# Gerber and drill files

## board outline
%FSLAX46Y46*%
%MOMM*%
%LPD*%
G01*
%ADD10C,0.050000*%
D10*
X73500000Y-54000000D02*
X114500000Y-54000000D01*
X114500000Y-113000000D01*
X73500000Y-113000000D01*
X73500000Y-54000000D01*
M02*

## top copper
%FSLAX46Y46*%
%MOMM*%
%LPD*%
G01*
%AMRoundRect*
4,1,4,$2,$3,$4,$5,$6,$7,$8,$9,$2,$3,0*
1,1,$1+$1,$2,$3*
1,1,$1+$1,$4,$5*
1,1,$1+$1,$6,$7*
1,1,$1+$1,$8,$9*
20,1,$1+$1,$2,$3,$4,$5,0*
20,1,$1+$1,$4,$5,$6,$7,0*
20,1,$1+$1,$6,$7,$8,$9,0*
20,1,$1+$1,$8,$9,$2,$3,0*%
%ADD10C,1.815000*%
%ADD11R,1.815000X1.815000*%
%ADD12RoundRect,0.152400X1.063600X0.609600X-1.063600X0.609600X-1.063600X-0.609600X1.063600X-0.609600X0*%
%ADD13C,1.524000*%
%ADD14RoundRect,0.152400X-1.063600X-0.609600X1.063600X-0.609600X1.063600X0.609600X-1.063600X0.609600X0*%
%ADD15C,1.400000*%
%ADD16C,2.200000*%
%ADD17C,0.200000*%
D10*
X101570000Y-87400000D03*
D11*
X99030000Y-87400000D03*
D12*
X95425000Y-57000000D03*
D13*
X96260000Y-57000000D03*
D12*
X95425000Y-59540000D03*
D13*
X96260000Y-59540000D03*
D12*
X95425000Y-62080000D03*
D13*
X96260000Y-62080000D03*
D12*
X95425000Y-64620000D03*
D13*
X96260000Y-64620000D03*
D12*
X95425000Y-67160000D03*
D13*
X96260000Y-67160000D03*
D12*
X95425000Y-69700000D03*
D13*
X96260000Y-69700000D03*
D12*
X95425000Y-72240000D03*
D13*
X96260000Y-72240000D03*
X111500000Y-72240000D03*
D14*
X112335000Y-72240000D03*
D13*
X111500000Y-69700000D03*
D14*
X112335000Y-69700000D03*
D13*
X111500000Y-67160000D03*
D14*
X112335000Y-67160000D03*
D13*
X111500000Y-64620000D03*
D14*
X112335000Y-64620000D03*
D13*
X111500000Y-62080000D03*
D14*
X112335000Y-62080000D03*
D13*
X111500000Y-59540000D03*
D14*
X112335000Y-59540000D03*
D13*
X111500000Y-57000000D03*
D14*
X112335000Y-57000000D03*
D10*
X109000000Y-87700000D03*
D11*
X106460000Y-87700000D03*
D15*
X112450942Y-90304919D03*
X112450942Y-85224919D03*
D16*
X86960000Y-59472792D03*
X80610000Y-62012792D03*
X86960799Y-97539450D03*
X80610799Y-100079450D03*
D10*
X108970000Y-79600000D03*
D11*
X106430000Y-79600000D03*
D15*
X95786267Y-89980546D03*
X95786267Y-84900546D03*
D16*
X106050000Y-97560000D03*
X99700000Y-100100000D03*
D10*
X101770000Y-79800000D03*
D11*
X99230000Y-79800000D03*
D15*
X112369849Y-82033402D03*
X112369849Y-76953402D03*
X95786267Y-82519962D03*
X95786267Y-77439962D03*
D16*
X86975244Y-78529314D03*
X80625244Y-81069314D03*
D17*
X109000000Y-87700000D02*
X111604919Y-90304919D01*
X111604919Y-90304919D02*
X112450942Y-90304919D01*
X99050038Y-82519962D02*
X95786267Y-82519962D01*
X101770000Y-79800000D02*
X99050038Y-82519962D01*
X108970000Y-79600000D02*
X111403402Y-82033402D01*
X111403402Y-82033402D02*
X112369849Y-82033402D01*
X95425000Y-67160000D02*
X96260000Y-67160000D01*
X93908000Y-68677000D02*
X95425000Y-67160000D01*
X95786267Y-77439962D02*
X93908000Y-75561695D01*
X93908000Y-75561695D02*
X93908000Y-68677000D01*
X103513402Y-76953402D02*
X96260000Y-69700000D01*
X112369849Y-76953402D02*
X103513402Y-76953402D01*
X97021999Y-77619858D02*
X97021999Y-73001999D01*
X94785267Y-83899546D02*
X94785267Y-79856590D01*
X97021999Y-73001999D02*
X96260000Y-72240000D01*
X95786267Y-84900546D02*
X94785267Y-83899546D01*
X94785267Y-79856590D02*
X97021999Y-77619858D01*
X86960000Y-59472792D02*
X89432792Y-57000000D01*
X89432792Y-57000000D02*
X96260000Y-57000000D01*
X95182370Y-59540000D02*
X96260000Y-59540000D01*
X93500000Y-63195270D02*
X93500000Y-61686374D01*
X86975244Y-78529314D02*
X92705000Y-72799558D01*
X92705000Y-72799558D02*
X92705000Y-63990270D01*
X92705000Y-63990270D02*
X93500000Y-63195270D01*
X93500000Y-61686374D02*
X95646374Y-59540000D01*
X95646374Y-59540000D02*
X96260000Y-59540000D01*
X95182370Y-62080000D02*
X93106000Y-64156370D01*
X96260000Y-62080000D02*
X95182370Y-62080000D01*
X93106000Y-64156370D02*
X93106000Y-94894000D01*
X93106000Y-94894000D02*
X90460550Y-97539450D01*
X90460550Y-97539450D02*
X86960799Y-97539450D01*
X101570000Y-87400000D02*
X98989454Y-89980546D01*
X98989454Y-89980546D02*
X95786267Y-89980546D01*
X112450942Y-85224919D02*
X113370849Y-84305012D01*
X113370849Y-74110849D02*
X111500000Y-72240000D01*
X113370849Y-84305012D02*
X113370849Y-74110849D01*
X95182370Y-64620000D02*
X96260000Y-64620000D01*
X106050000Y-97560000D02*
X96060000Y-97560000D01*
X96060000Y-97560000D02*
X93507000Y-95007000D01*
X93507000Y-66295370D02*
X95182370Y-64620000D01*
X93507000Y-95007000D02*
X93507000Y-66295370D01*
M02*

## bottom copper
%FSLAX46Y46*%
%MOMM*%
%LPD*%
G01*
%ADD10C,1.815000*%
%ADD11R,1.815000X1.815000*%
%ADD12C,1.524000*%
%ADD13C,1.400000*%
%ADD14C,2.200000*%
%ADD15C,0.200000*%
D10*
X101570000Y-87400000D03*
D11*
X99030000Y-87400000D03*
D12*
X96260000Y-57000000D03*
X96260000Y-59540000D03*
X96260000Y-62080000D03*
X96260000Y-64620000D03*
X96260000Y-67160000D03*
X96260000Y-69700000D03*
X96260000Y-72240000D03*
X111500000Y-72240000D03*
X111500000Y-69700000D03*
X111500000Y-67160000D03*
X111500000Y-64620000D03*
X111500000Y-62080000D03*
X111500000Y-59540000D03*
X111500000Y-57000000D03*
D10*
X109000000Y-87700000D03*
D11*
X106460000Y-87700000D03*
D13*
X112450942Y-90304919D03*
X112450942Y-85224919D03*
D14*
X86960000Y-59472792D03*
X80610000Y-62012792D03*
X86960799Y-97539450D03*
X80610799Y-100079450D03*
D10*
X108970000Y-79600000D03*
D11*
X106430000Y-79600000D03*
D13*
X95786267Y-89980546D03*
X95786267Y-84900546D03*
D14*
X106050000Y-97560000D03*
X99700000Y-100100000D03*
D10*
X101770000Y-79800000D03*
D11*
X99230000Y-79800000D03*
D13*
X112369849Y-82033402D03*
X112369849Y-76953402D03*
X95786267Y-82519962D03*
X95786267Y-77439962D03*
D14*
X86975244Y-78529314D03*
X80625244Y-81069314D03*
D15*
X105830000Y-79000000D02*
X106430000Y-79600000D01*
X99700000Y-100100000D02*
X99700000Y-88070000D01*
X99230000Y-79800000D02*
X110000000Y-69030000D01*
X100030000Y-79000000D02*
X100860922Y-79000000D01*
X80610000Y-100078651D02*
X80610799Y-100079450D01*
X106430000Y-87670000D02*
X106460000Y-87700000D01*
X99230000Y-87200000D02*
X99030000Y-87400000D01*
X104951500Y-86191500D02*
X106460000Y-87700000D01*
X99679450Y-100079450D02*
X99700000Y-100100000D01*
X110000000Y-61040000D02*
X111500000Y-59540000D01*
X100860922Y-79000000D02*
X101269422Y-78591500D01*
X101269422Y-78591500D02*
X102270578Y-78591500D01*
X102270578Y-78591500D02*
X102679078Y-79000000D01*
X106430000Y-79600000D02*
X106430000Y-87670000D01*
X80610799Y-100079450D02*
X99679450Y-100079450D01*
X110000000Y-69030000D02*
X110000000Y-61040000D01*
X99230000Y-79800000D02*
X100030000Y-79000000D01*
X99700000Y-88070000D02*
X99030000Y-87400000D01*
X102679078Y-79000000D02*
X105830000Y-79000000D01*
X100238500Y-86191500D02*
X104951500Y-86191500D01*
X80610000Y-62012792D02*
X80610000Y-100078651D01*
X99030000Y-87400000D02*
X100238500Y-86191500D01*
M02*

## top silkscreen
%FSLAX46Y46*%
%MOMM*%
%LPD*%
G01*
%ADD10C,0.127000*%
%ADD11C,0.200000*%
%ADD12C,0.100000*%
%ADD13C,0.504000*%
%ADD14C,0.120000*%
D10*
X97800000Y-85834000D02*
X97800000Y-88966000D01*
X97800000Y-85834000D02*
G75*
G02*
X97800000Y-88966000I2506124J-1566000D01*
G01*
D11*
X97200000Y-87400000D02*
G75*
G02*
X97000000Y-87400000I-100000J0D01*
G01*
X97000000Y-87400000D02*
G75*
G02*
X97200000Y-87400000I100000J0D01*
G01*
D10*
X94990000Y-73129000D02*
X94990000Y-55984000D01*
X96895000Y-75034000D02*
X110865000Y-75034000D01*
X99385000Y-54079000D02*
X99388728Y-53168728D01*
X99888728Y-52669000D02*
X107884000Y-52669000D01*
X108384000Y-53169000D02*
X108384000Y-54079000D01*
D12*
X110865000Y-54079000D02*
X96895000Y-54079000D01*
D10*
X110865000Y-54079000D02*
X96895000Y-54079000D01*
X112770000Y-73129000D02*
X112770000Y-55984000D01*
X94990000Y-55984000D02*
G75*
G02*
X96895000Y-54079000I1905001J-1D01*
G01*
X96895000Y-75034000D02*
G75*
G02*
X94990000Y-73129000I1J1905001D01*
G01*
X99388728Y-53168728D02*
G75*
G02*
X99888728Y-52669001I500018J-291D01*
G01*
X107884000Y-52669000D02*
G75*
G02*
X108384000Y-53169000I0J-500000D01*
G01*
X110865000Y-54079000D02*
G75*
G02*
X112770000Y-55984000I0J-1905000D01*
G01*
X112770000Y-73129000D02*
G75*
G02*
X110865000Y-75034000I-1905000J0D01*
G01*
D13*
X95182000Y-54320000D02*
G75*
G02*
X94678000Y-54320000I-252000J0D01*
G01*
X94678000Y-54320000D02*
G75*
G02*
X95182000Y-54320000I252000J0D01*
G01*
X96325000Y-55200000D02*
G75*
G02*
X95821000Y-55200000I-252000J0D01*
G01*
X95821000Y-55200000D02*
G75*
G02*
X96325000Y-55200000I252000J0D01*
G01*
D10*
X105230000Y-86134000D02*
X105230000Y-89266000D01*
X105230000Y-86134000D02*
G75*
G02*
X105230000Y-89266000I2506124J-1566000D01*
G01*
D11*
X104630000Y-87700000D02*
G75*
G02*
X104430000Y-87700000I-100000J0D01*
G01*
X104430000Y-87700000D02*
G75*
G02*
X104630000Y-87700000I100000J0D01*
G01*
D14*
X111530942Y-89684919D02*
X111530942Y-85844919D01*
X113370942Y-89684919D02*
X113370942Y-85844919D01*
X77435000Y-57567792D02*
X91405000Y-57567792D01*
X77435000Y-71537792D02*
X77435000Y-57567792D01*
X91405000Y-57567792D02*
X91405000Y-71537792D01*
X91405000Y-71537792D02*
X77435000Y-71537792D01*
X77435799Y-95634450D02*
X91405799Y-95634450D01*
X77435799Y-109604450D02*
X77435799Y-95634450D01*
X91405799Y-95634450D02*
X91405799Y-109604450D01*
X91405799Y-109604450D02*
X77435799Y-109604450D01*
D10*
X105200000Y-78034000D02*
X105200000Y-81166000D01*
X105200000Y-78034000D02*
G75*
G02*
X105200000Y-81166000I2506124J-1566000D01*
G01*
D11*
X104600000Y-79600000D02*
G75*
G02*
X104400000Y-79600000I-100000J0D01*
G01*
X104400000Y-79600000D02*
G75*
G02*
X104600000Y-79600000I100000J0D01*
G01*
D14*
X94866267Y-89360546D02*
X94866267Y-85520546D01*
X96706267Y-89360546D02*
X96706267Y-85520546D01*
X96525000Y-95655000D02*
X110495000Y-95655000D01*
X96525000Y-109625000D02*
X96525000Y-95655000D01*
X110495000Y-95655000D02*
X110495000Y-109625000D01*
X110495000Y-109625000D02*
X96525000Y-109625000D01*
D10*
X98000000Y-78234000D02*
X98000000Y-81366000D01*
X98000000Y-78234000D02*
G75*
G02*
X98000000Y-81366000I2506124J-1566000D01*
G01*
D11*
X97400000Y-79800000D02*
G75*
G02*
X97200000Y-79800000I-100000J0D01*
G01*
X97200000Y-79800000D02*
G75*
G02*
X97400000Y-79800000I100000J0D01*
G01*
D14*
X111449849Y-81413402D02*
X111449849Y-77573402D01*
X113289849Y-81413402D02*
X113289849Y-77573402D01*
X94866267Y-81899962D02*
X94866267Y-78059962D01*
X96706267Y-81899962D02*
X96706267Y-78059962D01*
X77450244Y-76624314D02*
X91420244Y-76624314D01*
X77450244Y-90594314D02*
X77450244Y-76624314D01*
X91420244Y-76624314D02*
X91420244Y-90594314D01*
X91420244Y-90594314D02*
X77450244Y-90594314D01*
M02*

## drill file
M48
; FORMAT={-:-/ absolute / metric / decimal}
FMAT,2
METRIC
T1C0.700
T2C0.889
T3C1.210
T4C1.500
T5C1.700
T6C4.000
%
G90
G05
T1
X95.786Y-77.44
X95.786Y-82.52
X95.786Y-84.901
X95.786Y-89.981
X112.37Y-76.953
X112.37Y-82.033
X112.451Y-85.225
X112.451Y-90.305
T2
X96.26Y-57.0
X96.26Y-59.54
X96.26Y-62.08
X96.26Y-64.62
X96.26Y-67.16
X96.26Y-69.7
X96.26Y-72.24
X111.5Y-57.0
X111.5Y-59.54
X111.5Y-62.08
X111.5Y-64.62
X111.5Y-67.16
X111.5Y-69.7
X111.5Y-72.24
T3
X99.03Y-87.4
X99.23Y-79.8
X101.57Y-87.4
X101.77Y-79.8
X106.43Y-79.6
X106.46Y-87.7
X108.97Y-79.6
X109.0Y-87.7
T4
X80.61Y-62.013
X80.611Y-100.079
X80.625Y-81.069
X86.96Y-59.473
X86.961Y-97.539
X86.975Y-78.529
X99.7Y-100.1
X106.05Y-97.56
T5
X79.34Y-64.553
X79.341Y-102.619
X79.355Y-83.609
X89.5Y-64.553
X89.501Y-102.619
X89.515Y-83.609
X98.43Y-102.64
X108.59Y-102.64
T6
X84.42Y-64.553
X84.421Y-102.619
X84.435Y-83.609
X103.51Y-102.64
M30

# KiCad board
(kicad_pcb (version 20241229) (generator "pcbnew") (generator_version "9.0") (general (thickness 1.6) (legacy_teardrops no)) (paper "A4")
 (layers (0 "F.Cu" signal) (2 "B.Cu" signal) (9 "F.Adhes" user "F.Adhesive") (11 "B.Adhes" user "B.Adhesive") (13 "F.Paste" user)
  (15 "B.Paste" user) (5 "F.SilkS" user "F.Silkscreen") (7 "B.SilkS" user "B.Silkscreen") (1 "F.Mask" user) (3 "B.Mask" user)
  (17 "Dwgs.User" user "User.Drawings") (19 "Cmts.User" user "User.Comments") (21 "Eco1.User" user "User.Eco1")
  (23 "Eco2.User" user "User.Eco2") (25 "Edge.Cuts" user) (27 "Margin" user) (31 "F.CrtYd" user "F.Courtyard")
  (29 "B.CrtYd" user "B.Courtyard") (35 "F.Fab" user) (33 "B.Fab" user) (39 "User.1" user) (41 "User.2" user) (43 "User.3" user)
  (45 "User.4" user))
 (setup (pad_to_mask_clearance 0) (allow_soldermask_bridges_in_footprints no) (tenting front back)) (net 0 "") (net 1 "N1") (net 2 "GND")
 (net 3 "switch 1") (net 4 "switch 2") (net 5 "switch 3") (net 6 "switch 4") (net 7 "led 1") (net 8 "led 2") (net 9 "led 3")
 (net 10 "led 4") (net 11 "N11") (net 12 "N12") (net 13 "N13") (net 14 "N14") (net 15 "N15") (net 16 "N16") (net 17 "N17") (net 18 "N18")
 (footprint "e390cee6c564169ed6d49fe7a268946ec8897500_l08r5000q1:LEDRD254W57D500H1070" (layer "F.Cu") (at 100.3 87.4)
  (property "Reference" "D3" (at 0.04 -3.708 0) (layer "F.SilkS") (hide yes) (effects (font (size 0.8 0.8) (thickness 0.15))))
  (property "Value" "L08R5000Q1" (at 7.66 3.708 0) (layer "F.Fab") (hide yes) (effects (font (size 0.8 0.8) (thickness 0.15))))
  (fp_line (start -2.5 -1.566) (end -2.5 1.566) (stroke (width 0.127) (type solid)) (layer "F.SilkS"))
  (fp_arc (start -2.5 -1.566) (mid 2.961291 0) (end -2.5 1.566) (stroke (width 0.127) (type solid)) (layer "F.SilkS"))
  (fp_circle (center -3.2 0) (end -3.1 0) (stroke (width 0.2) (type solid)) (fill no) (layer "F.SilkS"))
  (pad "A" thru_hole circle (at 1.27 0) (size 1.815 1.815) (drill 1.21) (layers "*.Cu" "*.Mask") (remove_unused_layers no) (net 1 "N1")
   (solder_mask_margin 0.102))
  (pad "C" thru_hole rect (at -1.27 0) (size 1.815 1.815) (drill 1.21) (layers "*.Cu" "*.Mask") (remove_unused_layers no) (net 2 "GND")
   (solder_mask_margin 0.102)))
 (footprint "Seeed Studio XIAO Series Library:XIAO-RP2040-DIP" (layer "F.Cu") (at 103.88 64.62)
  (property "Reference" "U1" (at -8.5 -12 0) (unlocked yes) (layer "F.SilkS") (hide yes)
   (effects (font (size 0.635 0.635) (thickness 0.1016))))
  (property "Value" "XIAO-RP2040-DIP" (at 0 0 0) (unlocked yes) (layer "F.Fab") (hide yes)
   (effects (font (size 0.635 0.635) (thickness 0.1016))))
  (fp_line (start -8.89 8.509) (end -8.89 -8.636) (stroke (width 0.127) (type solid)) (layer "F.SilkS"))
  (fp_line (start -6.985 10.414) (end 6.985 10.414) (stroke (width 0.127) (type solid)) (layer "F.SilkS"))
  (fp_line (start -4.495 -10.541) (end -4.491272 -11.451272) (stroke (width 0.127) (type solid)) (layer "F.SilkS"))
  (fp_line (start -3.991272 -11.951) (end 4.004 -11.951) (stroke (width 0.127) (type solid)) (layer "F.SilkS"))
  (fp_line (start 4.504 -11.451) (end 4.504 -10.541) (stroke (width 0.127) (type solid)) (layer "F.SilkS"))
  (fp_line (start 6.985 -10.541) (end -6.985 -10.541) (stroke (width 0.1) (type solid)) (layer "F.SilkS"))
  (fp_line (start 6.985 -10.541) (end -6.985 -10.541) (stroke (width 0.127) (type solid)) (layer "F.SilkS"))
  (fp_line (start 8.89 8.509) (end 8.89 -8.636) (stroke (width 0.127) (type solid)) (layer "F.SilkS"))
  (fp_arc (start -8.89 -8.636) (mid -8.332038 -9.983038) (end -6.985 -10.541) (stroke (width 0.127) (type solid)) (layer "F.SilkS"))
  (fp_arc (start -6.985 10.414) (mid -8.332038 9.856038) (end -8.89 8.509) (stroke (width 0.127) (type solid)) (layer "F.SilkS"))
  (fp_arc (start -4.491272 -11.451272) (mid -4.344724 -11.804644) (end -3.991272 -11.951) (stroke (width 0.127) (type default))
   (layer "F.SilkS"))
  (fp_arc (start 4.004 -11.951) (mid 4.357553 -11.804553) (end 4.504 -11.451) (stroke (width 0.127) (type default)) (layer "F.SilkS"))
  (fp_arc (start 6.985 -10.541) (mid 8.332038 -9.983038) (end 8.89 -8.636) (stroke (width 0.127) (type solid)) (layer "F.SilkS"))
  (fp_arc (start 8.89 8.509) (mid 8.332038 9.856038) (end 6.985 10.414) (stroke (width 0.127) (type solid)) (layer "F.SilkS"))
  (fp_circle (center -8.95 -10.3) (end -8.95 -10.554) (stroke (width 0.5) (type solid)) (fill yes) (layer "F.SilkS"))
  (fp_circle (center -7.807 -9.42) (end -7.807 -9.674) (stroke (width 0.5) (type solid)) (fill yes) (layer "F.SilkS"))
  (pad "1" smd roundrect (at -8.455 -7.62 180) (size 2.432 1.524) (layers "F.Cu" "F.Mask") (roundrect_rratio 0.1) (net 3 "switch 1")
   (thermal_bridge_angle 45))
  (pad "1" thru_hole circle (at -7.62 -7.62 180) (size 1.524 1.524) (drill 0.889) (layers "*.Cu" "*.Mask") (remove_unused_layers no)
   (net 3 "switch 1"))
  (pad "2" smd roundrect (at -8.455 -5.08 180) (size 2.432 1.524) (layers "F.Cu" "F.Mask") (roundrect_rratio 0.1) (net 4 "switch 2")
   (thermal_bridge_angle 45))
  (pad "2" thru_hole circle (at -7.62 -5.08 180) (size 1.524 1.524) (drill 0.889) (layers "*.Cu" "*.Mask") (remove_unused_layers no)
   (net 4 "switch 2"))
  (pad "3" smd roundrect (at -8.455 -2.54 180) (size 2.432 1.524) (layers "F.Cu" "F.Mask") (roundrect_rratio 0.1) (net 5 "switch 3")
   (thermal_bridge_angle 45))
  (pad "3" thru_hole circle (at -7.62 -2.54 180) (size 1.524 1.524) (drill 0.889) (layers "*.Cu" "*.Mask") (remove_unused_layers no)
   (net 5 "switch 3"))
  (pad "4" smd roundrect (at -8.455 0 180) (size 2.432 1.524) (layers "F.Cu" "F.Mask") (roundrect_rratio 0.1) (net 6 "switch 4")
   (thermal_bridge_angle 45))
  (pad "4" thru_hole circle (at -7.62 0 180) (size 1.524 1.524) (drill 0.889) (layers "*.Cu" "*.Mask") (remove_unused_layers no)
   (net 6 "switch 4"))
  (pad "5" smd roundrect (at -8.455 2.54 180) (size 2.432 1.524) (layers "F.Cu" "F.Mask") (roundrect_rratio 0.1) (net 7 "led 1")
   (thermal_bridge_angle 45))
  (pad "5" thru_hole circle (at -7.62 2.54 180) (size 1.524 1.524) (drill 0.889) (layers "*.Cu" "*.Mask") (remove_unused_layers no)
   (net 7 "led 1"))
  (pad "6" smd roundrect (at -8.455 5.08 180) (size 2.432 1.524) (layers "F.Cu" "F.Mask") (roundrect_rratio 0.1) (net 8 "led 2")
   (thermal_bridge_angle 45))
  (pad "6" thru_hole circle (at -7.62 5.08 180) (size 1.524 1.524) (drill 0.889) (layers "*.Cu" "*.Mask") (remove_unused_layers no)
   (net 8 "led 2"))
  (pad "7" smd roundrect (at -8.455 7.62 180) (size 2.432 1.524) (layers "F.Cu" "F.Mask") (roundrect_rratio 0.1) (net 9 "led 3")
   (thermal_bridge_angle 45))
  (pad "7" thru_hole circle (at -7.62 7.62 180) (size 1.524 1.524) (drill 0.889) (layers "*.Cu" "*.Mask") (remove_unused_layers no)
   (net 9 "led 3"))
  (pad "8" thru_hole circle (at 7.62 7.62) (size 1.524 1.524) (drill 0.889) (layers "*.Cu" "*.Mask") (remove_unused_layers no)
   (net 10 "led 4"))
  (pad "8" smd roundrect (at 8.455 7.62) (size 2.432 1.524) (layers "F.Cu" "F.Mask") (roundrect_rratio 0.1) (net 10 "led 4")
   (thermal_bridge_angle 45))
  (pad "9" thru_hole circle (at 7.62 5.08) (size 1.524 1.524) (drill 0.889) (layers "*.Cu" "*.Mask") (remove_unused_layers no)
   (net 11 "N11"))
  (pad "9" smd roundrect (at 8.455 5.08) (size 2.432 1.524) (layers "F.Cu" "F.Mask") (roundrect_rratio 0.1) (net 11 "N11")
   (thermal_bridge_angle 45))
  (pad "10" thru_hole circle (at 7.62 2.54) (size 1.524 1.524) (drill 0.889) (layers "*.Cu" "*.Mask") (remove_unused_layers no)
   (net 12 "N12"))
  (pad "10" smd roundrect (at 8.455 2.54) (size 2.432 1.524) (layers "F.Cu" "F.Mask") (roundrect_rratio 0.1) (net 12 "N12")
   (thermal_bridge_angle 45))
  (pad "11" thru_hole circle (at 7.62 0) (size 1.524 1.524) (drill 0.889) (layers "*.Cu" "*.Mask") (remove_unused_layers no) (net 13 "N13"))
  (pad "11" smd roundrect (at 8.455 0) (size 2.432 1.524) (layers "F.Cu" "F.Mask") (roundrect_rratio 0.1) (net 13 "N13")
   (thermal_bridge_angle 45))
  (pad "12" thru_hole circle (at 7.62 -2.54) (size 1.524 1.524) (drill 0.889) (layers "*.Cu" "*.Mask") (remove_unused_layers no)
   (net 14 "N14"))
  (pad "12" smd roundrect (at 8.455 -2.54) (size 2.432 1.524) (layers "F.Cu" "F.Mask") (roundrect_rratio 0.1) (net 14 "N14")
   (thermal_bridge_angle 45))
  (pad "13" thru_hole circle (at 7.62 -5.08) (size 1.524 1.524) (drill 0.889) (layers "*.Cu" "*.Mask") (remove_unused_layers no)
   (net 2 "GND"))
  (pad "13" smd roundrect (at 8.455 -5.08) (size 2.432 1.524) (layers "F.Cu" "F.Mask") (roundrect_rratio 0.1) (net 2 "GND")
   (thermal_bridge_angle 45))
  (pad "14" thru_hole circle (at 7.62 -7.62) (size 1.524 1.524) (drill 0.889) (layers "*.Cu" "*.Mask") (remove_unused_layers no)
   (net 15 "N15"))
  (pad "14" smd roundrect (at 8.455 -7.62) (size 2.432 1.524) (layers "F.Cu" "F.Mask") (roundrect_rratio 0.1) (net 15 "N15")
   (thermal_bridge_angle 45)))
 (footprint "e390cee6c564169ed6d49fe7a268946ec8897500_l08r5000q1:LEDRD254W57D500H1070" (layer "F.Cu") (at 107.73 87.7)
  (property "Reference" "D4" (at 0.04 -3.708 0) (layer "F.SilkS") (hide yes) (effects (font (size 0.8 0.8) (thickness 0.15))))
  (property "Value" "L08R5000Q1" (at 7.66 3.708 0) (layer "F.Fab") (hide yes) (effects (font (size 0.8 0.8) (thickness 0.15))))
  (fp_line (start -2.5 -1.566) (end -2.5 1.566) (stroke (width 0.127) (type solid)) (layer "F.SilkS"))
  (fp_arc (start -2.5 -1.566) (mid 2.961291 0) (end -2.5 1.566) (stroke (width 0.127) (type solid)) (layer "F.SilkS"))
  (fp_circle (center -3.2 0) (end -3.1 0) (stroke (width 0.2) (type solid)) (fill no) (layer "F.SilkS"))
  (pad "A" thru_hole circle (at 1.27 0) (size 1.815 1.815) (drill 1.21) (layers "*.Cu" "*.Mask") (remove_unused_layers no) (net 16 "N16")
   (solder_mask_margin 0.102))
  (pad "C" thru_hole rect (at -1.27 0) (size 1.815 1.815) (drill 1.21) (layers "*.Cu" "*.Mask") (remove_unused_layers no) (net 2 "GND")
   (solder_mask_margin 0.102)))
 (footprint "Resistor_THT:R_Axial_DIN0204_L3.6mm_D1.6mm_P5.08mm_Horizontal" (layer "F.Cu") (at 112.450942 90.304919 90)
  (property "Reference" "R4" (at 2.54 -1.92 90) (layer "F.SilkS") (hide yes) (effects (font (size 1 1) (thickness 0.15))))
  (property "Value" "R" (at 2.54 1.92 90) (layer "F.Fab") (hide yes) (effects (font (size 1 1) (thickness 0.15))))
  (fp_line (start 0.62 -0.92) (end 4.46 -0.92) (stroke (width 0.12) (type solid)) (layer "F.SilkS"))
  (fp_line (start 0.62 0.92) (end 4.46 0.92) (stroke (width 0.12) (type solid)) (layer "F.SilkS"))
  (pad "1" thru_hole circle (at 0 0 90) (size 1.4 1.4) (drill 0.7) (layers "*.Cu" "*.Mask") (remove_unused_layers no) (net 16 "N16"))
  (pad "2" thru_hole circle (at 5.08 0 90) (size 1.4 1.4) (drill 0.7) (layers "*.Cu" "*.Mask") (remove_unused_layers no) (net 10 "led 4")))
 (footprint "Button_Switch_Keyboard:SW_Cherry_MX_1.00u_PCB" (layer "F.Cu") (at 86.96 59.472792)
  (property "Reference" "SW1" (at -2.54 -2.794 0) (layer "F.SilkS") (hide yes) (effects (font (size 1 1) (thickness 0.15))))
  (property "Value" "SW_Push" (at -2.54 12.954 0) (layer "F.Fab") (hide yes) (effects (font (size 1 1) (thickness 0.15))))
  (fp_line (start -9.525 -1.905) (end 4.445 -1.905) (stroke (width 0.12) (type solid)) (layer "F.SilkS"))
  (fp_line (start -9.525 12.065) (end -9.525 -1.905) (stroke (width 0.12) (type solid)) (layer "F.SilkS"))
  (fp_line (start 4.445 -1.905) (end 4.445 12.065) (stroke (width 0.12) (type solid)) (layer "F.SilkS"))
  (fp_line (start 4.445 12.065) (end -9.525 12.065) (stroke (width 0.12) (type solid)) (layer "F.SilkS"))
  (pad "" np_thru_hole circle (at -7.62 5.08) (size 1.7 1.7) (drill 1.7) (layers "*.Cu" "*.Mask"))
  (pad "" np_thru_hole circle (at -2.54 5.08) (size 4 4) (drill 4) (layers "*.Cu" "*.Mask"))
  (pad "" np_thru_hole circle (at 2.54 5.08) (size 1.7 1.7) (drill 1.7) (layers "*.Cu" "*.Mask"))
  (pad "1" thru_hole circle (at 0 0) (size 2.2 2.2) (drill 1.5) (layers "*.Cu" "*.Mask") (remove_unused_layers no) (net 3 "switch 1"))
  (pad "2" thru_hole circle (at -6.35 2.54) (size 2.2 2.2) (drill 1.5) (layers "*.Cu" "*.Mask") (remove_unused_layers no) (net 2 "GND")))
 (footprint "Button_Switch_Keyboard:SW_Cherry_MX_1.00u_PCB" (layer "F.Cu") (at 86.960799 97.53945)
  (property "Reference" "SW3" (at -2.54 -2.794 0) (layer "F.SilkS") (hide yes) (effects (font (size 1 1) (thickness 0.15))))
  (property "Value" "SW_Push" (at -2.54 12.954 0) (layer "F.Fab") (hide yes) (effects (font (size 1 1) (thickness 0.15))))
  (fp_line (start -9.525 -1.905) (end 4.445 -1.905) (stroke (width 0.12) (type solid)) (layer "F.SilkS"))
  (fp_line (start -9.525 12.065) (end -9.525 -1.905) (stroke (width 0.12) (type solid)) (layer "F.SilkS"))
  (fp_line (start 4.445 -1.905) (end 4.445 12.065) (stroke (width 0.12) (type solid)) (layer "F.SilkS"))
  (fp_line (start 4.445 12.065) (end -9.525 12.065) (stroke (width 0.12) (type solid)) (layer "F.SilkS"))
  (pad "" np_thru_hole circle (at -7.62 5.08) (size 1.7 1.7) (drill 1.7) (layers "*.Cu" "*.Mask"))
  (pad "" np_thru_hole circle (at -2.54 5.08) (size 4 4) (drill 4) (layers "*.Cu" "*.Mask"))
  (pad "" np_thru_hole circle (at 2.54 5.08) (size 1.7 1.7) (drill 1.7) (layers "*.Cu" "*.Mask"))
  (pad "1" thru_hole circle (at 0 0) (size 2.2 2.2) (drill 1.5) (layers "*.Cu" "*.Mask") (remove_unused_layers no) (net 5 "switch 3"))
  (pad "2" thru_hole circle (at -6.35 2.54) (size 2.2 2.2) (drill 1.5) (layers "*.Cu" "*.Mask") (remove_unused_layers no) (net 2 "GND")))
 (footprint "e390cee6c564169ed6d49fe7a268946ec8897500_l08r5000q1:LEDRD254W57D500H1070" (layer "F.Cu") (at 107.7 79.6)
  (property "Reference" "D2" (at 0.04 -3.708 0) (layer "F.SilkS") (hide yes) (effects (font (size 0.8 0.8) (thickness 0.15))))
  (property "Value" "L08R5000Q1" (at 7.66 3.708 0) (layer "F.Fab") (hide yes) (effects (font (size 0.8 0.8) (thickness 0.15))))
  (fp_line (start -2.5 -1.566) (end -2.5 1.566) (stroke (width 0.127) (type solid)) (layer "F.SilkS"))
  (fp_arc (start -2.5 -1.566) (mid 2.961291 0) (end -2.5 1.566) (stroke (width 0.127) (type solid)) (layer "F.SilkS"))
  (fp_circle (center -3.2 0) (end -3.1 0) (stroke (width 0.2) (type solid)) (fill no) (layer "F.SilkS"))
  (pad "A" thru_hole circle (at 1.27 0) (size 1.815 1.815) (drill 1.21) (layers "*.Cu" "*.Mask") (remove_unused_layers no) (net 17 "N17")
   (solder_mask_margin 0.102))
  (pad "C" thru_hole rect (at -1.27 0) (size 1.815 1.815) (drill 1.21) (layers "*.Cu" "*.Mask") (remove_unused_layers no) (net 2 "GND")
   (solder_mask_margin 0.102)))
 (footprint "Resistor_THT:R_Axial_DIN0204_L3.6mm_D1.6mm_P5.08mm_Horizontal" (layer "F.Cu") (at 95.786267 89.980546 90)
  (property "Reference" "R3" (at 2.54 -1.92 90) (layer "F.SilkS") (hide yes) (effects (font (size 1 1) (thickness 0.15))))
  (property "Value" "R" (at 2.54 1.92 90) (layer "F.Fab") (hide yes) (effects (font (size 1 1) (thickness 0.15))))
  (fp_line (start 0.62 -0.92) (end 4.46 -0.92) (stroke (width 0.12) (type solid)) (layer "F.SilkS"))
  (fp_line (start 0.62 0.92) (end 4.46 0.92) (stroke (width 0.12) (type solid)) (layer "F.SilkS"))
  (pad "1" thru_hole circle (at 0 0 90) (size 1.4 1.4) (drill 0.7) (layers "*.Cu" "*.Mask") (remove_unused_layers no) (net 1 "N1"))
  (pad "2" thru_hole circle (at 5.08 0 90) (size 1.4 1.4) (drill 0.7) (layers "*.Cu" "*.Mask") (remove_unused_layers no) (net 9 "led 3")))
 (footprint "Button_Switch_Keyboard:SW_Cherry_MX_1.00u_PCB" (layer "F.Cu") (at 106.05 97.56)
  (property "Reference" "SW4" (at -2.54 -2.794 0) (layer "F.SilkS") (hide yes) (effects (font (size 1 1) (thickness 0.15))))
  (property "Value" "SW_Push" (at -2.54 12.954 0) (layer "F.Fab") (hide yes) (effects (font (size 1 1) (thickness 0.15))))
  (fp_line (start -9.525 -1.905) (end 4.445 -1.905) (stroke (width 0.12) (type solid)) (layer "F.SilkS"))
  (fp_line (start -9.525 12.065) (end -9.525 -1.905) (stroke (width 0.12) (type solid)) (layer "F.SilkS"))
  (fp_line (start 4.445 -1.905) (end 4.445 12.065) (stroke (width 0.12) (type solid)) (layer "F.SilkS"))
  (fp_line (start 4.445 12.065) (end -9.525 12.065) (stroke (width 0.12) (type solid)) (layer "F.SilkS"))
  (pad "" np_thru_hole circle (at -7.62 5.08) (size 1.7 1.7) (drill 1.7) (layers "*.Cu" "*.Mask"))
  (pad "" np_thru_hole circle (at -2.54 5.08) (size 4 4) (drill 4) (layers "*.Cu" "*.Mask"))
  (pad "" np_thru_hole circle (at 2.54 5.08) (size 1.7 1.7) (drill 1.7) (layers "*.Cu" "*.Mask"))
  (pad "1" thru_hole circle (at 0 0) (size 2.2 2.2) (drill 1.5) (layers "*.Cu" "*.Mask") (remove_unused_layers no) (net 6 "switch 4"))
  (pad "2" thru_hole circle (at -6.35 2.54) (size 2.2 2.2) (drill 1.5) (layers "*.Cu" "*.Mask") (remove_unused_layers no) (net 2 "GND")))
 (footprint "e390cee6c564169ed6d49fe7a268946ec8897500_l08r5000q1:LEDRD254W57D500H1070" (layer "F.Cu") (at 100.5 79.8)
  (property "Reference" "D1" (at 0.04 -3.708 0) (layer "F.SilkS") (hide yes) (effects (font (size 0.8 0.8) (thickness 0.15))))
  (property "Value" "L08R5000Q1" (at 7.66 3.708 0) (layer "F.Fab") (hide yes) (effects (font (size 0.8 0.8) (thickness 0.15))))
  (fp_line (start -2.5 -1.566) (end -2.5 1.566) (stroke (width 0.127) (type solid)) (layer "F.SilkS"))
  (fp_arc (start -2.5 -1.566) (mid 2.961291 0) (end -2.5 1.566) (stroke (width 0.127) (type solid)) (layer "F.SilkS"))
  (fp_circle (center -3.2 0) (end -3.1 0) (stroke (width 0.2) (type solid)) (fill no) (layer "F.SilkS"))
  (pad "A" thru_hole circle (at 1.27 0) (size 1.815 1.815) (drill 1.21) (layers "*.Cu" "*.Mask") (remove_unused_layers no) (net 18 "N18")
   (solder_mask_margin 0.102))
  (pad "C" thru_hole rect (at -1.27 0) (size 1.815 1.815) (drill 1.21) (layers "*.Cu" "*.Mask") (remove_unused_layers no) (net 2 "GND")
   (solder_mask_margin 0.102)))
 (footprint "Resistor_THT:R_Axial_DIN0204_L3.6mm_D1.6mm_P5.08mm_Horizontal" (layer "F.Cu") (at 112.369849 82.033402 90)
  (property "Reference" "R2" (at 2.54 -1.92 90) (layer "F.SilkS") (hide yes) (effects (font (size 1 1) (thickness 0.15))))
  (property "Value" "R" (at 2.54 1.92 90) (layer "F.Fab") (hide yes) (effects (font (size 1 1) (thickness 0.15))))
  (fp_line (start 0.62 -0.92) (end 4.46 -0.92) (stroke (width 0.12) (type solid)) (layer "F.SilkS"))
  (fp_line (start 0.62 0.92) (end 4.46 0.92) (stroke (width 0.12) (type solid)) (layer "F.SilkS"))
  (pad "1" thru_hole circle (at 0 0 90) (size 1.4 1.4) (drill 0.7) (layers "*.Cu" "*.Mask") (remove_unused_layers no) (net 17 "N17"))
  (pad "2" thru_hole circle (at 5.08 0 90) (size 1.4 1.4) (drill 0.7) (layers "*.Cu" "*.Mask") (remove_unused_layers no) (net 8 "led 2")))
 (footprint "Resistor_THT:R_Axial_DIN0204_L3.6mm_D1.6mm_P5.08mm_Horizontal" (layer "F.Cu") (at 95.786267 82.519962 90)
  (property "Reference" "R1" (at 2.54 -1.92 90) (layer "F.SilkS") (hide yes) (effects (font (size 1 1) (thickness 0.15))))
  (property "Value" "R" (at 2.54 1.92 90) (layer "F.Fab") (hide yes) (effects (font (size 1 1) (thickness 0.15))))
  (fp_line (start 0.62 -0.92) (end 4.46 -0.92) (stroke (width 0.12) (type solid)) (layer "F.SilkS"))
  (fp_line (start 0.62 0.92) (end 4.46 0.92) (stroke (width 0.12) (type solid)) (layer "F.SilkS"))
  (pad "1" thru_hole circle (at 0 0 90) (size 1.4 1.4) (drill 0.7) (layers "*.Cu" "*.Mask") (remove_unused_layers no) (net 18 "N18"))
  (pad "2" thru_hole circle (at 5.08 0 90) (size 1.4 1.4) (drill 0.7) (layers "*.Cu" "*.Mask") (remove_unused_layers no) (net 7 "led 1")))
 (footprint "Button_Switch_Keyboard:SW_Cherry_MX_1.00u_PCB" (layer "F.Cu") (at 86.975244 78.529314)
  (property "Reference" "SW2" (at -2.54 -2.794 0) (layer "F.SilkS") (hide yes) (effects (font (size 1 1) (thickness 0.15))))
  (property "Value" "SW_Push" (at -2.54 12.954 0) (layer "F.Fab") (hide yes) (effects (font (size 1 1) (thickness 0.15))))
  (fp_line (start -9.525 -1.905) (end 4.445 -1.905) (stroke (width 0.12) (type solid)) (layer "F.SilkS"))
  (fp_line (start -9.525 12.065) (end -9.525 -1.905) (stroke (width 0.12) (type solid)) (layer "F.SilkS"))
  (fp_line (start 4.445 -1.905) (end 4.445 12.065) (stroke (width 0.12) (type solid)) (layer "F.SilkS"))
  (fp_line (start 4.445 12.065) (end -9.525 12.065) (stroke (width 0.12) (type solid)) (layer "F.SilkS"))
  (pad "" np_thru_hole circle (at -7.62 5.08) (size 1.7 1.7) (drill 1.7) (layers "*.Cu" "*.Mask"))
  (pad "" np_thru_hole circle (at -2.54 5.08) (size 4 4) (drill 4) (layers "*.Cu" "*.Mask"))
  (pad "" np_thru_hole circle (at 2.54 5.08) (size 1.7 1.7) (drill 1.7) (layers "*.Cu" "*.Mask"))
  (pad "1" thru_hole circle (at 0 0) (size 2.2 2.2) (drill 1.5) (layers "*.Cu" "*.Mask") (remove_unused_layers no) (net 4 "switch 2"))
  (pad "2" thru_hole circle (at -6.35 2.54) (size 2.2 2.2) (drill 1.5) (layers "*.Cu" "*.Mask") (remove_unused_layers no) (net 2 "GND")))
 (gr_rect (start 73.5 54) (end 114.5 113) (stroke (width 0.05) (type default)) (fill no) (layer "Edge.Cuts"))
 (segment (start 109 87.7) (end 111.604919 90.304919) (width 0.2) (layer "F.Cu") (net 16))
 (segment (start 111.604919 90.304919) (end 112.450942 90.304919) (width 0.2) (layer "F.Cu") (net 16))
 (segment (start 105.83 79) (end 106.43 79.6) (width 0.2) (layer "B.Cu") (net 2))
 (segment (start 99.7 100.1) (end 99.7 88.07) (width 0.2) (layer "B.Cu") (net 2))
 (segment (start 99.23 79.8) (end 110 69.03) (width 0.2) (layer "B.Cu") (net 2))
 (segment (start 100.03 79) (end 100.860922 79) (width 0.2) (layer "B.Cu") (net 2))
 (segment (start 80.61 100.078651) (end 80.610799 100.07945) (width 0.2) (layer "B.Cu") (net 2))
 (segment (start 106.43 87.67) (end 106.46 87.7) (width 0.2) (layer "B.Cu") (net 2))
 (segment (start 99.23 87.2) (end 99.03 87.4) (width 0.2) (layer "B.Cu") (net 2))
 (segment (start 104.9515 86.1915) (end 106.46 87.7) (width 0.2) (layer "B.Cu") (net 2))
 (segment (start 99.67945 100.07945) (end 99.7 100.1) (width 0.2) (layer "B.Cu") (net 2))
 (segment (start 110 61.04) (end 111.5 59.54) (width 0.2) (layer "B.Cu") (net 2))
 (segment (start 100.860922 79) (end 101.269422 78.5915) (width 0.2) (layer "B.Cu") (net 2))
 (segment (start 101.269422 78.5915) (end 102.270578 78.5915) (width 0.2) (layer "B.Cu") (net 2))
 (segment (start 102.270578 78.5915) (end 102.679078 79) (width 0.2) (layer "B.Cu") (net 2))
 (segment (start 106.43 79.6) (end 106.43 87.67) (width 0.2) (layer "B.Cu") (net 2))
 (segment (start 80.610799 100.07945) (end 99.67945 100.07945) (width 0.2) (layer "B.Cu") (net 2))
 (segment (start 110 69.03) (end 110 61.04) (width 0.2) (layer "B.Cu") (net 2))
 (segment (start 99.23 79.8) (end 100.03 79) (width 0.2) (layer "B.Cu") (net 2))
 (segment (start 99.7 88.07) (end 99.03 87.4) (width 0.2) (layer "B.Cu") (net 2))
 (segment (start 102.679078 79) (end 105.83 79) (width 0.2) (layer "B.Cu") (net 2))
 (segment (start 100.2385 86.1915) (end 104.9515 86.1915) (width 0.2) (layer "B.Cu") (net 2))
 (segment (start 80.61 62.012792) (end 80.61 100.078651) (width 0.2) (layer "B.Cu") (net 2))
 (segment (start 99.03 87.4) (end 100.2385 86.1915) (width 0.2) (layer "B.Cu") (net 2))
 (segment (start 99.050038 82.519962) (end 95.786267 82.519962) (width 0.2) (layer "F.Cu") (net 18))
 (segment (start 101.77 79.8) (end 99.050038 82.519962) (width 0.2) (layer "F.Cu") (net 18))
 (segment (start 108.97 79.6) (end 111.403402 82.033402) (width 0.2) (layer "F.Cu") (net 17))
 (segment (start 111.403402 82.033402) (end 112.369849 82.033402) (width 0.2) (layer "F.Cu") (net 17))
 (segment (start 95.425 67.16) (end 96.26 67.16) (width 0.2) (layer "F.Cu") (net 7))
 (segment (start 93.908 68.677) (end 95.425 67.16) (width 0.2) (layer "F.Cu") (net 7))
 (segment (start 95.786267 77.439962) (end 93.908 75.561695) (width 0.2) (layer "F.Cu") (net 7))
 (segment (start 93.908 75.561695) (end 93.908 68.677) (width 0.2) (layer "F.Cu") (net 7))
 (segment (start 103.513402 76.953402) (end 96.26 69.7) (width 0.2) (layer "F.Cu") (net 8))
 (segment (start 112.369849 76.953402) (end 103.513402 76.953402) (width 0.2) (layer "F.Cu") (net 8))
 (segment (start 97.021999 77.619858) (end 97.021999 73.001999) (width 0.2) (layer "F.Cu") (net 9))
 (segment (start 94.785267 83.899546) (end 94.785267 79.85659) (width 0.2) (layer "F.Cu") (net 9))
 (segment (start 97.021999 73.001999) (end 96.26 72.24) (width 0.2) (layer "F.Cu") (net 9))
 (segment (start 95.786267 84.900546) (end 94.785267 83.899546) (width 0.2) (layer "F.Cu") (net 9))
 (segment (start 94.785267 79.85659) (end 97.021999 77.619858) (width 0.2) (layer "F.Cu") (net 9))
 (segment (start 86.96 59.472792) (end 89.432792 57) (width 0.2) (layer "F.Cu") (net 3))
 (segment (start 89.432792 57) (end 96.26 57) (width 0.2) (layer "F.Cu") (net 3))
 (segment (start 95.18237 59.54) (end 96.26 59.54) (width 0.2) (layer "F.Cu") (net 4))
 (segment (start 93.5 63.19527) (end 93.5 61.686374) (width 0.2) (layer "F.Cu") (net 4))
 (segment (start 86.975244 78.529314) (end 92.705 72.799558) (width 0.2) (layer "F.Cu") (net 4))
 (segment (start 92.705 72.799558) (end 92.705 63.99027) (width 0.2) (layer "F.Cu") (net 4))
 (segment (start 92.705 63.99027) (end 93.5 63.19527) (width 0.2) (layer "F.Cu") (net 4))
 (segment (start 93.5 61.686374) (end 95.646374 59.54) (width 0.2) (layer "F.Cu") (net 4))
 (segment (start 95.646374 59.54) (end 96.26 59.54) (width 0.2) (layer "F.Cu") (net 4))
 (segment (start 95.18237 62.08) (end 93.106 64.15637) (width 0.2) (layer "F.Cu") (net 5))
 (segment (start 96.26 62.08) (end 95.18237 62.08) (width 0.2) (layer "F.Cu") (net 5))
 (segment (start 93.106 64.15637) (end 93.106 94.894) (width 0.2) (layer "F.Cu") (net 5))
 (segment (start 93.106 94.894) (end 90.46055 97.53945) (width 0.2) (layer "F.Cu") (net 5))
 (segment (start 90.46055 97.53945) (end 86.960799 97.53945) (width 0.2) (layer "F.Cu") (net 5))
 (segment (start 101.57 87.4) (end 98.989454 89.980546) (width 0.2) (layer "F.Cu") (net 1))
 (segment (start 98.989454 89.980546) (end 95.786267 89.980546) (width 0.2) (layer "F.Cu") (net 1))
 (segment (start 112.450942 85.224919) (end 113.370849 84.305012) (width 0.2) (layer "F.Cu") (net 10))
 (segment (start 113.370849 74.110849) (end 111.5 72.24) (width 0.2) (layer "F.Cu") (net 10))
 (segment (start 113.370849 84.305012) (end 113.370849 74.110849) (width 0.2) (layer "F.Cu") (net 10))
 (segment (start 95.18237 64.62) (end 96.26 64.62) (width 0.2) (layer "F.Cu") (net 6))
 (segment (start 106.05 97.56) (end 96.06 97.56) (width 0.2) (layer "F.Cu") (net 6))
 (segment (start 96.06 97.56) (end 93.507 95.007) (width 0.2) (layer "F.Cu") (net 6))
 (segment (start 93.507 66.29537) (end 95.18237 64.62) (width 0.2) (layer "F.Cu") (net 6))
 (segment (start 93.507 95.007) (end 93.507 66.29537) (width 0.2) (layer "F.Cu") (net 6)))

